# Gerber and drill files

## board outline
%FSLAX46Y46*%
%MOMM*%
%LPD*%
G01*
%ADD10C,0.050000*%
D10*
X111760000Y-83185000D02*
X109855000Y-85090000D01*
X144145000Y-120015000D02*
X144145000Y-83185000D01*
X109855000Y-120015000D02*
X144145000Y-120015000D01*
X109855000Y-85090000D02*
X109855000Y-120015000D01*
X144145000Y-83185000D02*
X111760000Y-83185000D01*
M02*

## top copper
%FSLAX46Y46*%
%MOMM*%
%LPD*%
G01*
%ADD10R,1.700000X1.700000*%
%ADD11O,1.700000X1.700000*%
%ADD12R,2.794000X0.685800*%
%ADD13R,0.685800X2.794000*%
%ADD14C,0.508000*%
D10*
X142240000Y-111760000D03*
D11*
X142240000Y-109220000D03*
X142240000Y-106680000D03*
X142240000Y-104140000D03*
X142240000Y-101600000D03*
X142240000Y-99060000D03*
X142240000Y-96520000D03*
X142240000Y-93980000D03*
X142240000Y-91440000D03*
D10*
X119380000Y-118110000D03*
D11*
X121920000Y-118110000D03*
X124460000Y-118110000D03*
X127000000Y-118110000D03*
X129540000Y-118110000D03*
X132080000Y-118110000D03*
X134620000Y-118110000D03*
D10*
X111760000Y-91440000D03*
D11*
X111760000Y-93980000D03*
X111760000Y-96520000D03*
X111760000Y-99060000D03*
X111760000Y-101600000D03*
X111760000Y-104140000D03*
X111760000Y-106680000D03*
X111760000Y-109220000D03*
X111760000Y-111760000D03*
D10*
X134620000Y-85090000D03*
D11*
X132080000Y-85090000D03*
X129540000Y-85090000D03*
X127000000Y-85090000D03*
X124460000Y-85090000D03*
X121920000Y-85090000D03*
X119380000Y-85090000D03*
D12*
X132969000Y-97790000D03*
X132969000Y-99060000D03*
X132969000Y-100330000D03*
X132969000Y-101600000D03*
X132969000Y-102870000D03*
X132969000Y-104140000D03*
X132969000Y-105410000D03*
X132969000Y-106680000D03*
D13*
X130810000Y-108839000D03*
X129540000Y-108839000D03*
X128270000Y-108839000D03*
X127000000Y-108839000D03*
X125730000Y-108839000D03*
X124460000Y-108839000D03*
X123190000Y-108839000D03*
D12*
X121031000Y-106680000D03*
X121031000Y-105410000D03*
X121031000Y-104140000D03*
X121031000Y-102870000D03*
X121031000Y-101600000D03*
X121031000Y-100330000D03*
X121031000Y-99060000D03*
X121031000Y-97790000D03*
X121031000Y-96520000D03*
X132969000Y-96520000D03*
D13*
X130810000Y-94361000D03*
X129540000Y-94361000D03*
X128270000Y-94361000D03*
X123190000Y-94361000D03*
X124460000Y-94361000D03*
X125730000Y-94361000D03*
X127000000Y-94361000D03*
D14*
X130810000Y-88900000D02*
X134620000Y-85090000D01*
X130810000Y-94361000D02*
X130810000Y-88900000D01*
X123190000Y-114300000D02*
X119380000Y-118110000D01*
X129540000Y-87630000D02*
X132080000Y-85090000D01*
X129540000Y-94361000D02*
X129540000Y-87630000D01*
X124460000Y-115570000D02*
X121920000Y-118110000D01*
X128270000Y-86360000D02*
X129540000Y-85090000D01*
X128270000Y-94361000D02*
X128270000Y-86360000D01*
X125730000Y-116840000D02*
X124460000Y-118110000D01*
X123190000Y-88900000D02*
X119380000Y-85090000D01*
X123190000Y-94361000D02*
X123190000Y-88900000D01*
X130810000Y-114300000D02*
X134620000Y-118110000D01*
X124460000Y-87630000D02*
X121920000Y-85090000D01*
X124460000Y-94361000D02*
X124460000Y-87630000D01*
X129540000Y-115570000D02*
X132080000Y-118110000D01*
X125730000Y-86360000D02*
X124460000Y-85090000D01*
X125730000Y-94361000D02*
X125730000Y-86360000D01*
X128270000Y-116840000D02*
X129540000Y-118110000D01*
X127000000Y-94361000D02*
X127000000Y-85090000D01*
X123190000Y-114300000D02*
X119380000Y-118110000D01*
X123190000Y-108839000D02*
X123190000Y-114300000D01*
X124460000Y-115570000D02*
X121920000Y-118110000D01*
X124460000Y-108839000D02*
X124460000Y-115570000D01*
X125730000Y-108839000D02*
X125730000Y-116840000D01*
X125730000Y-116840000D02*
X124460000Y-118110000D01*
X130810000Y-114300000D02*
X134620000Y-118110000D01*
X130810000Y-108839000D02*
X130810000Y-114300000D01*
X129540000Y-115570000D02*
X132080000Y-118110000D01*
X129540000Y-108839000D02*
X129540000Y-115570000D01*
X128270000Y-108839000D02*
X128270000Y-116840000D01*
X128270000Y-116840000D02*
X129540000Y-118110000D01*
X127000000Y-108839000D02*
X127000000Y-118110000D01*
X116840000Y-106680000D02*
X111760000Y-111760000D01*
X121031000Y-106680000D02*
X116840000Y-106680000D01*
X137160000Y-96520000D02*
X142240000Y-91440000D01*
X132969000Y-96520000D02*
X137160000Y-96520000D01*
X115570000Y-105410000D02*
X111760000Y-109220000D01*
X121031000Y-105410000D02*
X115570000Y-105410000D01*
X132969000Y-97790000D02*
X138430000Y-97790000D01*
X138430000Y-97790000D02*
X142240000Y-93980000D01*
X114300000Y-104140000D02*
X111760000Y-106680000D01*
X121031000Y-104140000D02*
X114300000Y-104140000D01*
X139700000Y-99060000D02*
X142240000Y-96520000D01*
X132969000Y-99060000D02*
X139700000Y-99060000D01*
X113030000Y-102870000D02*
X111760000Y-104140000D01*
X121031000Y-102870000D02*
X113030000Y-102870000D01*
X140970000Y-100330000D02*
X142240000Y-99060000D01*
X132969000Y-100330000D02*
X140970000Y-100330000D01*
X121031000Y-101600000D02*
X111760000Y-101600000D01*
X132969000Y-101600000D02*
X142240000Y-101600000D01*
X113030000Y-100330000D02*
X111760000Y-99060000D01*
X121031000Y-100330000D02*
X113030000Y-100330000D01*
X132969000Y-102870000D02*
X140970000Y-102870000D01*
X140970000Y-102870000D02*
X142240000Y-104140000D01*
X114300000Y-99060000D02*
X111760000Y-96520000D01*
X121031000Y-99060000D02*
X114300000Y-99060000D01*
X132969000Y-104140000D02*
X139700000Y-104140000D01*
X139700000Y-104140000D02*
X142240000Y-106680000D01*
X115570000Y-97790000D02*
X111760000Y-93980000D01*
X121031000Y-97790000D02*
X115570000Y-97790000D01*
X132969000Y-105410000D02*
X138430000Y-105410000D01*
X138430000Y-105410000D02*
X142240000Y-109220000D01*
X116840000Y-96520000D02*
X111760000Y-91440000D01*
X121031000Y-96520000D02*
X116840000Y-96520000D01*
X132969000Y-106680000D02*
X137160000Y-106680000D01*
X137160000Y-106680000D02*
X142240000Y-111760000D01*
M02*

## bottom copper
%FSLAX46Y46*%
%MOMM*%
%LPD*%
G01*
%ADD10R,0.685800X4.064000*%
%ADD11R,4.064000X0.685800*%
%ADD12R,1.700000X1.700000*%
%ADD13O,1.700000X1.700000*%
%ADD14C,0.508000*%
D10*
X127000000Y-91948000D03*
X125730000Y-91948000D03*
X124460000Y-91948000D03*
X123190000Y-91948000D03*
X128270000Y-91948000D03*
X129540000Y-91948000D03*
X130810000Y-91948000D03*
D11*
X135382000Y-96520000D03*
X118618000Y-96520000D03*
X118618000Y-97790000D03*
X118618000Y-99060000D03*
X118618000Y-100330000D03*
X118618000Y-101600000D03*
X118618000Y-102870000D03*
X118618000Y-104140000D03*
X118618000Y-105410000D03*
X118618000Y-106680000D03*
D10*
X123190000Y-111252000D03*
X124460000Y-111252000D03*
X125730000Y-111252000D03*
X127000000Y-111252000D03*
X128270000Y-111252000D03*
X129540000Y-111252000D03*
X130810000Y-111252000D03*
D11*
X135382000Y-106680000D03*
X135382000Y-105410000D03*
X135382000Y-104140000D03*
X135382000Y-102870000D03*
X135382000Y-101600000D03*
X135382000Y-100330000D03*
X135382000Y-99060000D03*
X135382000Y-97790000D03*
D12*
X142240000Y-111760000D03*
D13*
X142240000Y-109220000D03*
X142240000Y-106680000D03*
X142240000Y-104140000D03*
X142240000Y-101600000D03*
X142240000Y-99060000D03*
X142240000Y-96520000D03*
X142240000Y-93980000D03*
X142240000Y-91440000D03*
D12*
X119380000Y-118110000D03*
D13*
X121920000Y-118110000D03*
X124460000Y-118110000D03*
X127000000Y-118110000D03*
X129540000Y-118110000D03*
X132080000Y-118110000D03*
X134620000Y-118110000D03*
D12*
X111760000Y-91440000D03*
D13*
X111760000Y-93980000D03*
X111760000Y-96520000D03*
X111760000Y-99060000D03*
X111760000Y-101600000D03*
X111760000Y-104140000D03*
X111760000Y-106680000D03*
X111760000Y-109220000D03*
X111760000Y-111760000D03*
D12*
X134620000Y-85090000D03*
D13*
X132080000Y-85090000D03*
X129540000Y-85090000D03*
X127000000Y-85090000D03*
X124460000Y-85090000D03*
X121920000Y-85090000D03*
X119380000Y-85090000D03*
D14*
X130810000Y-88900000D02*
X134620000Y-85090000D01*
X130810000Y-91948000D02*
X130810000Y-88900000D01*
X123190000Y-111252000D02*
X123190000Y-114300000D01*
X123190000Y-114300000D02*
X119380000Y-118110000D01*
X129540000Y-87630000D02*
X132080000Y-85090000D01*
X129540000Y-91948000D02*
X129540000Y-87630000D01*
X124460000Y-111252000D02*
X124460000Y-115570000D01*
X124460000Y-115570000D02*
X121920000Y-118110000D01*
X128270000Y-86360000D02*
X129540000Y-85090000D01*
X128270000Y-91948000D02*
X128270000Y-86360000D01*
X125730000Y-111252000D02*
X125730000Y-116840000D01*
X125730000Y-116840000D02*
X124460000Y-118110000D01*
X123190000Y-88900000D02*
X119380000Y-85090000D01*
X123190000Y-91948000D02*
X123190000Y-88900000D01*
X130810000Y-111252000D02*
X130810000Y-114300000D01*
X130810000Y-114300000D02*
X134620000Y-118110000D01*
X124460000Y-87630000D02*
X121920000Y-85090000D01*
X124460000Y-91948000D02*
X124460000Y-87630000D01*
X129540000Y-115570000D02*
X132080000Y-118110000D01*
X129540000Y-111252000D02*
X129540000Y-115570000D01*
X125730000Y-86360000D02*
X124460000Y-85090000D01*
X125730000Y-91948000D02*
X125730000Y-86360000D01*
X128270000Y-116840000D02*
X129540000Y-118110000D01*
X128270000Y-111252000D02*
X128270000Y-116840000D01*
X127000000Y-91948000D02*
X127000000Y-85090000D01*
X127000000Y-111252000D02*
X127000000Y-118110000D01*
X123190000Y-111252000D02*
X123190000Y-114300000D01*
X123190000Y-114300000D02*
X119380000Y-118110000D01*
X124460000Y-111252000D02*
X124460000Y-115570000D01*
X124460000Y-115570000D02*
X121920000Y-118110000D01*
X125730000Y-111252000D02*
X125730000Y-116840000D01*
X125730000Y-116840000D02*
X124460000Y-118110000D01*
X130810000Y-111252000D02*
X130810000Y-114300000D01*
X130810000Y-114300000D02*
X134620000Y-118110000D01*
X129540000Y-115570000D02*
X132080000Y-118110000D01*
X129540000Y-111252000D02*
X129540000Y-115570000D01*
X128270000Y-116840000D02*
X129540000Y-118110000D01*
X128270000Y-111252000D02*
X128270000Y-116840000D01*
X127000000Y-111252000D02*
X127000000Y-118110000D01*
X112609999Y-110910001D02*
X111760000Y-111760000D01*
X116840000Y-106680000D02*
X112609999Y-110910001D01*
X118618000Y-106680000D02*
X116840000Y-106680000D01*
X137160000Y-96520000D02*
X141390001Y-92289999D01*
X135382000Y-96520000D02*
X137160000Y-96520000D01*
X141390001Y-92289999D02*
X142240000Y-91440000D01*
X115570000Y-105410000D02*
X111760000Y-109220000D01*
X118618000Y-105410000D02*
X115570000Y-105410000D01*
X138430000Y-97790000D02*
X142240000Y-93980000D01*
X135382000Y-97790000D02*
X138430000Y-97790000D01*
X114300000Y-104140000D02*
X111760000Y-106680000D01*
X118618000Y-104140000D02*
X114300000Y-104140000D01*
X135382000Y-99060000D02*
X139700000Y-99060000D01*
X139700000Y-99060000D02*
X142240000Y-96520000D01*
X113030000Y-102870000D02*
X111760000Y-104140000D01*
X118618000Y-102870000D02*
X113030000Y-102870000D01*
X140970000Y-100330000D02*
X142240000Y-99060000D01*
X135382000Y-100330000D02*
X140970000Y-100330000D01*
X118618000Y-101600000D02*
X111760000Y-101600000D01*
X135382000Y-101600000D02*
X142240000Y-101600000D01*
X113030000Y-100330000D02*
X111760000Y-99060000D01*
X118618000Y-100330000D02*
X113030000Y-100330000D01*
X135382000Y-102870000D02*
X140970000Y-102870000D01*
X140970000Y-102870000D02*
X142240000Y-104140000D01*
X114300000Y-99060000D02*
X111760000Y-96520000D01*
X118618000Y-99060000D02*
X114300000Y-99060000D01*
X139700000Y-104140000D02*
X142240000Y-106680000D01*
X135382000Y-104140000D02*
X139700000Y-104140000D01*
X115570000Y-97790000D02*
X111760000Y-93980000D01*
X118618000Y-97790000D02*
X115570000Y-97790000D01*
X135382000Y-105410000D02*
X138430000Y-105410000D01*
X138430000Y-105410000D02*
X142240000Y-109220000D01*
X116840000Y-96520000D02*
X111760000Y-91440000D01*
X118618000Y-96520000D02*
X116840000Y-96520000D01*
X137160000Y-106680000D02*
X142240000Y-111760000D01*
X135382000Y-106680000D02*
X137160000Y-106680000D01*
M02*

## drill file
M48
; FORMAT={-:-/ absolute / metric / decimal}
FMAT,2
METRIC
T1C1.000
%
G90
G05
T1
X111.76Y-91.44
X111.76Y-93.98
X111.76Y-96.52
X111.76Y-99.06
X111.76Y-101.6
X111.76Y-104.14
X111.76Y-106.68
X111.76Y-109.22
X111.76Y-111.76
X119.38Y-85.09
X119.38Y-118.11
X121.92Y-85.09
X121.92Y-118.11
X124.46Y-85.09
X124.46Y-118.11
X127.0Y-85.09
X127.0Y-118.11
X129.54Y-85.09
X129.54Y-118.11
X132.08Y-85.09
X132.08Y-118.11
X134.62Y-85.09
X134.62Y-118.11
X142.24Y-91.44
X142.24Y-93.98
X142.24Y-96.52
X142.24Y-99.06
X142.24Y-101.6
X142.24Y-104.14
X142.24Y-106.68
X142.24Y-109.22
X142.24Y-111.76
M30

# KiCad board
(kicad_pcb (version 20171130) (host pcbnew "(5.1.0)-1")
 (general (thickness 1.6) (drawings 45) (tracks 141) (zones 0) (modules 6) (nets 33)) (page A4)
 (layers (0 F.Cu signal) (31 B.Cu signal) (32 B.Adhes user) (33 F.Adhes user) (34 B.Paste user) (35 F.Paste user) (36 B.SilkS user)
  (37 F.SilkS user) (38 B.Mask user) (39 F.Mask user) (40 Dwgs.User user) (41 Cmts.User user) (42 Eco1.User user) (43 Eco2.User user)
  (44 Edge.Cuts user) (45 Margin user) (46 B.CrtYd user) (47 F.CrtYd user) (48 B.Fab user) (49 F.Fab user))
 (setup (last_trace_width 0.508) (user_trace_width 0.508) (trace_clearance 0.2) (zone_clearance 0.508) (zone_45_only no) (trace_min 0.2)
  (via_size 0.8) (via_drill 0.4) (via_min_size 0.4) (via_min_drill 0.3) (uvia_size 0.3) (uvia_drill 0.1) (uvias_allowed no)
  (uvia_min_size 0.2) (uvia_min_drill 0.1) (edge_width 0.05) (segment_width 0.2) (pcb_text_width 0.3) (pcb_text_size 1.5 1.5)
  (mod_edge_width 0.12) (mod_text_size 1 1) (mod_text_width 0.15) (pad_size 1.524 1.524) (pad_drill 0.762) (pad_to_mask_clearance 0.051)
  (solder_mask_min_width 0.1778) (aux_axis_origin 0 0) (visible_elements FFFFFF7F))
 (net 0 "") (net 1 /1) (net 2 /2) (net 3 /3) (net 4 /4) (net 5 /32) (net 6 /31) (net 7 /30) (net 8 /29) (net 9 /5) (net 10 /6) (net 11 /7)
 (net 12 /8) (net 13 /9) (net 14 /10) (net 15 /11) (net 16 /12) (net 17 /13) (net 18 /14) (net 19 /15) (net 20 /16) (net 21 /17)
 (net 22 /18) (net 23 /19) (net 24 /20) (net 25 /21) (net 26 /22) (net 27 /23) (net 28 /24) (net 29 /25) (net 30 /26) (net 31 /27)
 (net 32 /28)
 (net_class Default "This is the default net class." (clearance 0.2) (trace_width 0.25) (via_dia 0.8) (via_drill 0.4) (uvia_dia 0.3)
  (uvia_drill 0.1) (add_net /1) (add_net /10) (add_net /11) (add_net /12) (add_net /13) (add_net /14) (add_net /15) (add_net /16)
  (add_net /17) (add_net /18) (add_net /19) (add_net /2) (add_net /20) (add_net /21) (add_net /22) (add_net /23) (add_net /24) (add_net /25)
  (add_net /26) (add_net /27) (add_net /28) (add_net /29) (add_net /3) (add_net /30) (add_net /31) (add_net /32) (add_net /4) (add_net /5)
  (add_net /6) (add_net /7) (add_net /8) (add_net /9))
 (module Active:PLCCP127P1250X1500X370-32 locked (layer B.Cu) (at 127 101.6 180)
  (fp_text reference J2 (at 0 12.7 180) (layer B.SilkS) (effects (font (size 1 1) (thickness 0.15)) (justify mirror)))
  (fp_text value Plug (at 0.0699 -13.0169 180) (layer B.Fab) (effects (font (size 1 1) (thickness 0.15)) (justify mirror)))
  (pad 1 smd rect (at 0 9.652 180) (size 0.6858 4.064) (layers B.Cu B.Paste B.Mask) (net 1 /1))
  (pad 2 smd rect (at 1.27 9.652 180) (size 0.6858 4.064) (layers B.Cu B.Paste B.Mask) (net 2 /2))
  (pad 3 smd rect (at 2.54 9.652 180) (size 0.6858 4.064) (layers B.Cu B.Paste B.Mask) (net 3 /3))
  (pad 4 smd rect (at 3.81 9.652 180) (size 0.6858 4.064) (layers B.Cu B.Paste B.Mask) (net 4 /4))
  (pad 32 smd rect (at -1.27 9.652 180) (size 0.6858 4.064) (layers B.Cu B.Paste B.Mask) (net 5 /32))
  (pad 31 smd rect (at -2.54 9.652 180) (size 0.6858 4.064) (layers B.Cu B.Paste B.Mask) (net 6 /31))
  (pad 30 smd rect (at -3.81 9.652 180) (size 0.6858 4.064) (layers B.Cu B.Paste B.Mask) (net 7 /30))
  (pad 29 smd rect (at -8.382 5.08 270) (size 0.6858 4.064) (layers B.Cu B.Paste B.Mask) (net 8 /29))
  (pad 5 smd rect (at 8.382 5.08 270) (size 0.6858 4.064) (layers B.Cu B.Paste B.Mask) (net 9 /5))
  (pad 6 smd rect (at 8.382 3.81 270) (size 0.6858 4.064) (layers B.Cu B.Paste B.Mask) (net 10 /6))
  (pad 7 smd rect (at 8.382 2.54 270) (size 0.6858 4.064) (layers B.Cu B.Paste B.Mask) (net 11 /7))
  (pad 8 smd rect (at 8.382 1.27 270) (size 0.6858 4.064) (layers B.Cu B.Paste B.Mask) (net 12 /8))
  (pad 9 smd rect (at 8.382 0 270) (size 0.6858 4.064) (layers B.Cu B.Paste B.Mask) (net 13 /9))
  (pad 10 smd rect (at 8.382 -1.27 270) (size 0.6858 4.064) (layers B.Cu B.Paste B.Mask) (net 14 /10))
  (pad 11 smd rect (at 8.382 -2.54 270) (size 0.6858 4.064) (layers B.Cu B.Paste B.Mask) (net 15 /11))
  (pad 12 smd rect (at 8.382 -3.81 270) (size 0.6858 4.064) (layers B.Cu B.Paste B.Mask) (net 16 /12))
  (pad 13 smd rect (at 8.382 -5.08 270) (size 0.6858 4.064) (layers B.Cu B.Paste B.Mask) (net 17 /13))
  (pad 14 smd rect (at 3.81 -9.652 180) (size 0.6858 4.064) (layers B.Cu B.Paste B.Mask) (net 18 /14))
  (pad 15 smd rect (at 2.54 -9.652 180) (size 0.6858 4.064) (layers B.Cu B.Paste B.Mask) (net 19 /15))
  (pad 16 smd rect (at 1.27 -9.652 180) (size 0.6858 4.064) (layers B.Cu B.Paste B.Mask) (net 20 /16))
  (pad 17 smd rect (at 0 -9.652 180) (size 0.6858 4.064) (layers B.Cu B.Paste B.Mask) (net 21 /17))
  (pad 18 smd rect (at -1.27 -9.652 180) (size 0.6858 4.064) (layers B.Cu B.Paste B.Mask) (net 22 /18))
  (pad 19 smd rect (at -2.54 -9.652 180) (size 0.6858 4.064) (layers B.Cu B.Paste B.Mask) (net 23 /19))
  (pad 20 smd rect (at -3.81 -9.652 180) (size 0.6858 4.064) (layers B.Cu B.Paste B.Mask) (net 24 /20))
  (pad 21 smd rect (at -8.382 -5.08 270) (size 0.6858 4.064) (layers B.Cu B.Paste B.Mask) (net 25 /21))
  (pad 22 smd rect (at -8.382 -3.81 270) (size 0.6858 4.064) (layers B.Cu B.Paste B.Mask) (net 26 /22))
  (pad 23 smd rect (at -8.382 -2.54 270) (size 0.6858 4.064) (layers B.Cu B.Paste B.Mask) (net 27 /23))
  (pad 24 smd rect (at -8.382 -1.27 270) (size 0.6858 4.064) (layers B.Cu B.Paste B.Mask) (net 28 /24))
  (pad 25 smd rect (at -8.382 0 270) (size 0.6858 4.064) (layers B.Cu B.Paste B.Mask) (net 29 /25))
  (pad 26 smd rect (at -8.382 1.27 270) (size 0.6858 4.064) (layers B.Cu B.Paste B.Mask) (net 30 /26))
  (pad 27 smd rect (at -8.382 2.54 270) (size 0.6858 4.064) (layers B.Cu B.Paste B.Mask) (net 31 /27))
  (pad 28 smd rect (at -8.382 3.81 270) (size 0.6858 4.064) (layers B.Cu B.Paste B.Mask) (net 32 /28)))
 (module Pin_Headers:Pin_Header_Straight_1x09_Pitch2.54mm (layer F.Cu) (at 142.24 111.76 180)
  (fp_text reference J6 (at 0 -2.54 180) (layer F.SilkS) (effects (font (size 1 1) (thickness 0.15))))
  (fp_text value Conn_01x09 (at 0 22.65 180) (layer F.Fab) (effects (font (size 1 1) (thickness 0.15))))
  (pad 1 thru_hole rect (at 0 0 180) (size 1.7 1.7) (drill 1) (layers *.Cu *.Mask) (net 25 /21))
  (pad 2 thru_hole oval (at 0 2.54 180) (size 1.7 1.7) (drill 1) (layers *.Cu *.Mask) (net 26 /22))
  (pad 3 thru_hole oval (at 0 5.08 180) (size 1.7 1.7) (drill 1) (layers *.Cu *.Mask) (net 27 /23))
  (pad 4 thru_hole oval (at 0 7.62 180) (size 1.7 1.7) (drill 1) (layers *.Cu *.Mask) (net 28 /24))
  (pad 5 thru_hole oval (at 0 10.16 180) (size 1.7 1.7) (drill 1) (layers *.Cu *.Mask) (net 29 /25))
  (pad 6 thru_hole oval (at 0 12.7 180) (size 1.7 1.7) (drill 1) (layers *.Cu *.Mask) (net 30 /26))
  (pad 7 thru_hole oval (at 0 15.24 180) (size 1.7 1.7) (drill 1) (layers *.Cu *.Mask) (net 31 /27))
  (pad 8 thru_hole oval (at 0 17.78 180) (size 1.7 1.7) (drill 1) (layers *.Cu *.Mask) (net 32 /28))
  (pad 9 thru_hole oval (at 0 20.32 180) (size 1.7 1.7) (drill 1) (layers *.Cu *.Mask) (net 8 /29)))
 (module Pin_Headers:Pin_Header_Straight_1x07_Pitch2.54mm (layer F.Cu) (at 119.38 118.11 90)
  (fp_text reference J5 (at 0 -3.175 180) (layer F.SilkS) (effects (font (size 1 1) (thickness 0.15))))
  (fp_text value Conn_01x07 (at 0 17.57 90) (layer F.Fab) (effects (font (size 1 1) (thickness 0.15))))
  (pad 1 thru_hole rect (at 0 0 90) (size 1.7 1.7) (drill 1) (layers *.Cu *.Mask) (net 18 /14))
  (pad 2 thru_hole oval (at 0 2.54 90) (size 1.7 1.7) (drill 1) (layers *.Cu *.Mask) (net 19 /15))
  (pad 3 thru_hole oval (at 0 5.08 90) (size 1.7 1.7) (drill 1) (layers *.Cu *.Mask) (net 20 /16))
  (pad 4 thru_hole oval (at 0 7.62 90) (size 1.7 1.7) (drill 1) (layers *.Cu *.Mask) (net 21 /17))
  (pad 5 thru_hole oval (at 0 10.16 90) (size 1.7 1.7) (drill 1) (layers *.Cu *.Mask) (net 22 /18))
  (pad 6 thru_hole oval (at 0 12.7 90) (size 1.7 1.7) (drill 1) (layers *.Cu *.Mask) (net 23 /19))
  (pad 7 thru_hole oval (at 0 15.24 90) (size 1.7 1.7) (drill 1) (layers *.Cu *.Mask) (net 24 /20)))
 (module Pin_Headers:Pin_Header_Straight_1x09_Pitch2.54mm (layer F.Cu) (at 111.76 91.44)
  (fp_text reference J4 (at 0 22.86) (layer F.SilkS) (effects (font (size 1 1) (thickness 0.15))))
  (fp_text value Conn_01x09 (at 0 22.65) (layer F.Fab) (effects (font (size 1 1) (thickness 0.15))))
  (pad 1 thru_hole rect (at 0 0) (size 1.7 1.7) (drill 1) (layers *.Cu *.Mask) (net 9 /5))
  (pad 2 thru_hole oval (at 0 2.54) (size 1.7 1.7) (drill 1) (layers *.Cu *.Mask) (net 10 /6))
  (pad 3 thru_hole oval (at 0 5.08) (size 1.7 1.7) (drill 1) (layers *.Cu *.Mask) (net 11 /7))
  (pad 4 thru_hole oval (at 0 7.62) (size 1.7 1.7) (drill 1) (layers *.Cu *.Mask) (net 12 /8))
  (pad 5 thru_hole oval (at 0 10.16) (size 1.7 1.7) (drill 1) (layers *.Cu *.Mask) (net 13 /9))
  (pad 6 thru_hole oval (at 0 12.7) (size 1.7 1.7) (drill 1) (layers *.Cu *.Mask) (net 14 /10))
  (pad 7 thru_hole oval (at 0 15.24) (size 1.7 1.7) (drill 1) (layers *.Cu *.Mask) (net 15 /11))
  (pad 8 thru_hole oval (at 0 17.78) (size 1.7 1.7) (drill 1) (layers *.Cu *.Mask) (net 16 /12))
  (pad 9 thru_hole oval (at 0 20.32) (size 1.7 1.7) (drill 1) (layers *.Cu *.Mask) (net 17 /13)))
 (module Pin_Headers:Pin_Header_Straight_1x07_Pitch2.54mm (layer F.Cu) (at 134.62 85.09 270)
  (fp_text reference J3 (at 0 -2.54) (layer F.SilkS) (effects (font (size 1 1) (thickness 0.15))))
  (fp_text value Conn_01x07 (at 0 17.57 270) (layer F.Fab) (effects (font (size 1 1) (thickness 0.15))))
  (pad 1 thru_hole rect (at 0 0 270) (size 1.7 1.7) (drill 1) (layers *.Cu *.Mask) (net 7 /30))
  (pad 2 thru_hole oval (at 0 2.54 270) (size 1.7 1.7) (drill 1) (layers *.Cu *.Mask) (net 6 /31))
  (pad 3 thru_hole oval (at 0 5.08 270) (size 1.7 1.7) (drill 1) (layers *.Cu *.Mask) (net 5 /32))
  (pad 4 thru_hole oval (at 0 7.62 270) (size 1.7 1.7) (drill 1) (layers *.Cu *.Mask) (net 1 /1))
  (pad 5 thru_hole oval (at 0 10.16 270) (size 1.7 1.7) (drill 1) (layers *.Cu *.Mask) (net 2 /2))
  (pad 6 thru_hole oval (at 0 12.7 270) (size 1.7 1.7) (drill 1) (layers *.Cu *.Mask) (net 3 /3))
  (pad 7 thru_hole oval (at 0 15.24 270) (size 1.7 1.7) (drill 1) (layers *.Cu *.Mask) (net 4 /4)))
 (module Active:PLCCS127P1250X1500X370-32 (layer F.Cu) (at 127 101.6)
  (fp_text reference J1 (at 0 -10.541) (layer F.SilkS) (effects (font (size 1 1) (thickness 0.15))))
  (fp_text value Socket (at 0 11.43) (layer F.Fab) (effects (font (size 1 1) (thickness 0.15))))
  (pad 28 smd rect (at 5.969 -3.81 90) (size 0.6858 2.794) (layers F.Cu F.Paste F.Mask) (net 32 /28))
  (pad 27 smd rect (at 5.969 -2.54 90) (size 0.6858 2.794) (layers F.Cu F.Paste F.Mask) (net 31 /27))
  (pad 26 smd rect (at 5.969 -1.27 90) (size 0.6858 2.794) (layers F.Cu F.Paste F.Mask) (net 30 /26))
  (pad 25 smd rect (at 5.969 0 90) (size 0.6858 2.794) (layers F.Cu F.Paste F.Mask) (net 29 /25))
  (pad 24 smd rect (at 5.969 1.27 90) (size 0.6858 2.794) (layers F.Cu F.Paste F.Mask) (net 28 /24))
  (pad 23 smd rect (at 5.969 2.54 90) (size 0.6858 2.794) (layers F.Cu F.Paste F.Mask) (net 27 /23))
  (pad 22 smd rect (at 5.969 3.81 90) (size 0.6858 2.794) (layers F.Cu F.Paste F.Mask) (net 26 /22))
  (pad 21 smd rect (at 5.969 5.08 90) (size 0.6858 2.794) (layers F.Cu F.Paste F.Mask) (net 25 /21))
  (pad 20 smd rect (at 3.81 7.239) (size 0.6858 2.794) (layers F.Cu F.Paste F.Mask) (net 24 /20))
  (pad 19 smd rect (at 2.54 7.239) (size 0.6858 2.794) (layers F.Cu F.Paste F.Mask) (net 23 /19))
  (pad 18 smd rect (at 1.27 7.239) (size 0.6858 2.794) (layers F.Cu F.Paste F.Mask) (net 22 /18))
  (pad 17 smd rect (at 0 7.239) (size 0.6858 2.794) (layers F.Cu F.Paste F.Mask) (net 21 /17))
  (pad 16 smd rect (at -1.27 7.239) (size 0.6858 2.794) (layers F.Cu F.Paste F.Mask) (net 20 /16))
  (pad 15 smd rect (at -2.54 7.239) (size 0.6858 2.794) (layers F.Cu F.Paste F.Mask) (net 19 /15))
  (pad 14 smd rect (at -3.81 7.239) (size 0.6858 2.794) (layers F.Cu F.Paste F.Mask) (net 18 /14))
  (pad 13 smd rect (at -5.969 5.08 90) (size 0.6858 2.794) (layers F.Cu F.Paste F.Mask) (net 17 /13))
  (pad 12 smd rect (at -5.969 3.81 90) (size 0.6858 2.794) (layers F.Cu F.Paste F.Mask) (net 16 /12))
  (pad 11 smd rect (at -5.969 2.54 90) (size 0.6858 2.794) (layers F.Cu F.Paste F.Mask) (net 15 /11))
  (pad 10 smd rect (at -5.969 1.27 90) (size 0.6858 2.794) (layers F.Cu F.Paste F.Mask) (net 14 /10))
  (pad 9 smd rect (at -5.969 0 90) (size 0.6858 2.794) (layers F.Cu F.Paste F.Mask) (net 13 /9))
  (pad 8 smd rect (at -5.969 -1.27 90) (size 0.6858 2.794) (layers F.Cu F.Paste F.Mask) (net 12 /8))
  (pad 7 smd rect (at -5.969 -2.54 90) (size 0.6858 2.794) (layers F.Cu F.Paste F.Mask) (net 11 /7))
  (pad 6 smd rect (at -5.969 -3.81 90) (size 0.6858 2.794) (layers F.Cu F.Paste F.Mask) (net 10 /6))
  (pad 5 smd rect (at -5.969 -5.08 90) (size 0.6858 2.794) (layers F.Cu F.Paste F.Mask) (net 9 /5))
  (pad 29 smd rect (at 5.969 -5.08 90) (size 0.6858 2.794) (layers F.Cu F.Paste F.Mask) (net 8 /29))
  (pad 30 smd rect (at 3.81 -7.239) (size 0.6858 2.794) (layers F.Cu F.Paste F.Mask) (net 7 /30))
  (pad 31 smd rect (at 2.54 -7.239) (size 0.6858 2.794) (layers F.Cu F.Paste F.Mask) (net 6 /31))
  (pad 32 smd rect (at 1.27 -7.239) (size 0.6858 2.794) (layers F.Cu F.Paste F.Mask) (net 5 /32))
  (pad 4 smd rect (at -3.81 -7.239) (size 0.6858 2.794) (layers F.Cu F.Paste F.Mask) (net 4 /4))
  (pad 3 smd rect (at -2.54 -7.239) (size 0.6858 2.794) (layers F.Cu F.Paste F.Mask) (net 3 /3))
  (pad 2 smd rect (at -1.27 -7.239) (size 0.6858 2.794) (layers F.Cu F.Paste F.Mask) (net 2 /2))
  (pad 1 smd rect (at 0 -7.239) (size 0.6858 2.794) (layers F.Cu F.Paste F.Mask) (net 1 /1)))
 (gr_line (start 111.76 83.185) (end 109.855 85.09) (layer Edge.Cuts) (width 0.05))
 (gr_line (start 144.145 120.015) (end 144.145 83.185) (layer Edge.Cuts) (width 0.05))
 (gr_line (start 109.855 120.015) (end 144.145 120.015) (layer Edge.Cuts) (width 0.05))
 (gr_line (start 109.855 85.09) (end 109.855 120.015) (layer Edge.Cuts) (width 0.05))
 (gr_line (start 144.145 83.185) (end 111.76 83.185) (layer Edge.Cuts) (width 0.05))
 (segment (start 130.81 88.9) (end 134.62 85.09) (width 0.508) (layer F.Cu) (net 7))
 (segment (start 130.81 94.361) (end 130.81 88.9) (width 0.508) (layer F.Cu) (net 7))
 (segment (start 130.81 88.9) (end 134.62 85.09) (width 0.508) (layer B.Cu) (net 7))
 (segment (start 130.81 91.948) (end 130.81 88.9) (width 0.508) (layer B.Cu) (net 7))
 (segment (start 123.19 114.3) (end 119.38 118.11) (width 0.508) (layer F.Cu) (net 18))
 (segment (start 123.19 111.252) (end 123.19 114.3) (width 0.508) (layer B.Cu) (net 18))
 (segment (start 123.19 114.3) (end 119.38 118.11) (width 0.508) (layer B.Cu) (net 18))
 (segment (start 129.54 87.63) (end 132.08 85.09) (width 0.508) (layer F.Cu) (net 6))
 (segment (start 129.54 94.361) (end 129.54 87.63) (width 0.508) (layer F.Cu) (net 6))
 (segment (start 129.54 87.63) (end 132.08 85.09) (width 0.508) (layer B.Cu) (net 6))
 (segment (start 129.54 91.948) (end 129.54 87.63) (width 0.508) (layer B.Cu) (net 6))
 (segment (start 124.46 111.252) (end 124.46 115.57) (width 0.508) (layer B.Cu) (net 19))
 (segment (start 124.46 115.57) (end 121.92 118.11) (width 0.508) (layer B.Cu) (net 19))
 (segment (start 124.46 115.57) (end 121.92 118.11) (width 0.508) (layer F.Cu) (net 19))
 (segment (start 128.27 86.36) (end 129.54 85.09) (width 0.508) (layer F.Cu) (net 5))
 (segment (start 128.27 94.361) (end 128.27 86.36) (width 0.508) (layer F.Cu) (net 5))
 (segment (start 128.27 86.36) (end 129.54 85.09) (width 0.508) (layer B.Cu) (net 5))
 (segment (start 128.27 91.948) (end 128.27 86.36) (width 0.508) (layer B.Cu) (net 5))
 (segment (start 125.73 116.84) (end 124.46 118.11) (width 0.508) (layer F.Cu) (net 20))
 (segment (start 125.73 111.252) (end 125.73 116.84) (width 0.508) (layer B.Cu) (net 20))
 (segment (start 125.73 116.84) (end 124.46 118.11) (width 0.508) (layer B.Cu) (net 20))
 (segment (start 123.19 88.9) (end 119.38 85.09) (width 0.508) (layer F.Cu) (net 4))
 (segment (start 123.19 94.361) (end 123.19 88.9) (width 0.508) (layer F.Cu) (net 4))
 (segment (start 123.19 88.9) (end 119.38 85.09) (width 0.508) (layer B.Cu) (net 4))
 (segment (start 123.19 91.948) (end 123.19 88.9) (width 0.508) (layer B.Cu) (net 4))
 (segment (start 130.81 114.3) (end 134.62 118.11) (width 0.508) (layer F.Cu) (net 24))
 (segment (start 130.81 111.252) (end 130.81 114.3) (width 0.508) (layer B.Cu) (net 24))
 (segment (start 130.81 114.3) (end 134.62 118.11) (width 0.508) (layer B.Cu) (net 24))
 (segment (start 124.46 87.63) (end 121.92 85.09) (width 0.508) (layer F.Cu) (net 3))
 (segment (start 124.46 94.361) (end 124.46 87.63) (width 0.508) (layer F.Cu) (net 3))
 (segment (start 124.46 87.63) (end 121.92 85.09) (width 0.508) (layer B.Cu) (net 3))
 (segment (start 124.46 91.948) (end 124.46 87.63) (width 0.508) (layer B.Cu) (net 3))
 (segment (start 129.54 115.57) (end 132.08 118.11) (width 0.508) (layer F.Cu) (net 23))
 (segment (start 129.54 115.57) (end 132.08 118.11) (width 0.508) (layer B.Cu) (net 23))
 (segment (start 129.54 111.252) (end 129.54 115.57) (width 0.508) (layer B.Cu) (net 23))
 (segment (start 125.73 86.36) (end 124.46 85.09) (width 0.508) (layer F.Cu) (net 2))
 (segment (start 125.73 94.361) (end 125.73 86.36) (width 0.508) (layer F.Cu) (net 2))
 (segment (start 125.73 86.36) (end 124.46 85.09) (width 0.508) (layer B.Cu) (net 2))
 (segment (start 125.73 91.948) (end 125.73 86.36) (width 0.508) (layer B.Cu) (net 2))
 (segment (start 128.27 116.84) (end 129.54 118.11) (width 0.508) (layer B.Cu) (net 22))
 (segment (start 128.27 111.252) (end 128.27 116.84) (width 0.508) (layer B.Cu) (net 22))
 (segment (start 128.27 116.84) (end 129.54 118.11) (width 0.508) (layer F.Cu) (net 22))
 (segment (start 127 94.361) (end 127 85.09) (width 0.508) (layer F.Cu) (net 1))
 (segment (start 127 91.948) (end 127 85.09) (width 0.508) (layer B.Cu) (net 1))
 (segment (start 127 111.252) (end 127 118.11) (width 0.508) (layer B.Cu) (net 21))
 (segment (start 123.19 114.3) (end 119.38 118.11) (width 0.508) (layer F.Cu) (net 18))
 (segment (start 123.19 108.839) (end 123.19 114.3) (width 0.508) (layer F.Cu) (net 18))
 (segment (start 123.19 111.252) (end 123.19 114.3) (width 0.508) (layer B.Cu) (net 18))
 (segment (start 123.19 114.3) (end 119.38 118.11) (width 0.508) (layer B.Cu) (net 18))
 (segment (start 124.46 111.252) (end 124.46 115.57) (width 0.508) (layer B.Cu) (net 19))
 (segment (start 124.46 115.57) (end 121.92 118.11) (width 0.508) (layer B.Cu) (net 19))
 (segment (start 124.46 115.57) (end 121.92 118.11) (width 0.508) (layer F.Cu) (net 19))
 (segment (start 124.46 108.839) (end 124.46 115.57) (width 0.508) (layer F.Cu) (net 19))
 (segment (start 125.73 108.839) (end 125.73 116.84) (width 0.508) (layer F.Cu) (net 20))
 (segment (start 125.73 116.84) (end 124.46 118.11) (width 0.508) (layer F.Cu) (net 20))
 (segment (start 125.73 111.252) (end 125.73 116.84) (width 0.508) (layer B.Cu) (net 20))
 (segment (start 125.73 116.84) (end 124.46 118.11) (width 0.508) (layer B.Cu) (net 20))
 (segment (start 130.81 114.3) (end 134.62 118.11) (width 0.508) (layer F.Cu) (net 24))
 (segment (start 130.81 108.839) (end 130.81 114.3) (width 0.508) (layer F.Cu) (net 24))
 (segment (start 130.81 111.252) (end 130.81 114.3) (width 0.508) (layer B.Cu) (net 24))
 (segment (start 130.81 114.3) (end 134.62 118.11) (width 0.508) (layer B.Cu) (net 24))
 (segment (start 129.54 115.57) (end 132.08 118.11) (width 0.508) (layer F.Cu) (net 23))
 (segment (start 129.54 108.839) (end 129.54 115.57) (width 0.508) (layer F.Cu) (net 23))
 (segment (start 129.54 115.57) (end 132.08 118.11) (width 0.508) (layer B.Cu) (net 23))
 (segment (start 129.54 111.252) (end 129.54 115.57) (width 0.508) (layer B.Cu) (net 23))
 (segment (start 128.27 116.84) (end 129.54 118.11) (width 0.508) (layer B.Cu) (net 22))
 (segment (start 128.27 111.252) (end 128.27 116.84) (width 0.508) (layer B.Cu) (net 22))
 (segment (start 128.27 108.839) (end 128.27 116.84) (width 0.508) (layer F.Cu) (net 22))
 (segment (start 128.27 116.84) (end 129.54 118.11) (width 0.508) (layer F.Cu) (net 22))
 (segment (start 127 111.252) (end 127 118.11) (width 0.508) (layer B.Cu) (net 21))
 (segment (start 127 108.839) (end 127 118.11) (width 0.508) (layer F.Cu) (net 21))
 (segment (start 116.84 106.68) (end 111.76 111.76) (width 0.508) (layer F.Cu) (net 17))
 (segment (start 121.031 106.68) (end 116.84 106.68) (width 0.508) (layer F.Cu) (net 17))
 (segment (start 112.609999 110.910001) (end 111.76 111.76) (width 0.508) (layer B.Cu) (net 17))
 (segment (start 116.84 106.68) (end 112.609999 110.910001) (width 0.508) (layer B.Cu) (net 17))
 (segment (start 118.618 106.68) (end 116.84 106.68) (width 0.508) (layer B.Cu) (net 17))
 (segment (start 137.16 96.52) (end 141.390001 92.289999) (width 0.508) (layer B.Cu) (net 8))
 (segment (start 135.382 96.52) (end 137.16 96.52) (width 0.508) (layer B.Cu) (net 8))
 (segment (start 141.390001 92.289999) (end 142.24 91.44) (width 0.508) (layer B.Cu) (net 8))
 (segment (start 137.16 96.52) (end 142.24 91.44) (width 0.508) (layer F.Cu) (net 8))
 (segment (start 132.969 96.52) (end 137.16 96.52) (width 0.508) (layer F.Cu) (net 8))
 (segment (start 115.57 105.41) (end 111.76 109.22) (width 0.508) (layer F.Cu) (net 16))
 (segment (start 121.031 105.41) (end 115.57 105.41) (width 0.508) (layer F.Cu) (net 16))
 (segment (start 115.57 105.41) (end 111.76 109.22) (width 0.508) (layer B.Cu) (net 16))
 (segment (start 118.618 105.41) (end 115.57 105.41) (width 0.508) (layer B.Cu) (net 16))
 (segment (start 132.969 97.79) (end 138.43 97.79) (width 0.508) (layer F.Cu) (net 32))
 (segment (start 138.43 97.79) (end 142.24 93.98) (width 0.508) (layer F.Cu) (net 32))
 (segment (start 138.43 97.79) (end 142.24 93.98) (width 0.508) (layer B.Cu) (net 32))
 (segment (start 135.382 97.79) (end 138.43 97.79) (width 0.508) (layer B.Cu) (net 32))
 (segment (start 114.3 104.14) (end 111.76 106.68) (width 0.508) (layer F.Cu) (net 15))
 (segment (start 121.031 104.14) (end 114.3 104.14) (width 0.508) (layer F.Cu) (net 15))
 (segment (start 114.3 104.14) (end 111.76 106.68) (width 0.508) (layer B.Cu) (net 15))
 (segment (start 118.618 104.14) (end 114.3 104.14) (width 0.508) (layer B.Cu) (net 15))
 (segment (start 135.382 99.06) (end 139.7 99.06) (width 0.508) (layer B.Cu) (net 31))
 (segment (start 139.7 99.06) (end 142.24 96.52) (width 0.508) (layer B.Cu) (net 31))
 (segment (start 139.7 99.06) (end 142.24 96.52) (width 0.508) (layer F.Cu) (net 31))
 (segment (start 132.969 99.06) (end 139.7 99.06) (width 0.508) (layer F.Cu) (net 31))
 (segment (start 113.03 102.87) (end 111.76 104.14) (width 0.508) (layer F.Cu) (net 14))
 (segment (start 121.031 102.87) (end 113.03 102.87) (width 0.508) (layer F.Cu) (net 14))
 (segment (start 113.03 102.87) (end 111.76 104.14) (width 0.508) (layer B.Cu) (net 14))
 (segment (start 118.618 102.87) (end 113.03 102.87) (width 0.508) (layer B.Cu) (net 14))
 (segment (start 140.97 100.33) (end 142.24 99.06) (width 0.508) (layer B.Cu) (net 30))
 (segment (start 135.382 100.33) (end 140.97 100.33) (width 0.508) (layer B.Cu) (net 30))
 (segment (start 140.97 100.33) (end 142.24 99.06) (width 0.508) (layer F.Cu) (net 30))
 (segment (start 132.969 100.33) (end 140.97 100.33) (width 0.508) (layer F.Cu) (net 30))
 (segment (start 121.031 101.6) (end 111.76 101.6) (width 0.508) (layer F.Cu) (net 13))
 (segment (start 118.618 101.6) (end 111.76 101.6) (width 0.508) (layer B.Cu) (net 13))
 (segment (start 132.969 101.6) (end 142.24 101.6) (width 0.508) (layer F.Cu) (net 29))
 (segment (start 135.382 101.6) (end 142.24 101.6) (width 0.508) (layer B.Cu) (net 29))
 (segment (start 113.03 100.33) (end 111.76 99.06) (width 0.508) (layer F.Cu) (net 12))
 (segment (start 121.031 100.33) (end 113.03 100.33) (width 0.508) (layer F.Cu) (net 12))
 (segment (start 113.03 100.33) (end 111.76 99.06) (width 0.508) (layer B.Cu) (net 12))
 (segment (start 118.618 100.33) (end 113.03 100.33) (width 0.508) (layer B.Cu) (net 12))
 (segment (start 132.969 102.87) (end 140.97 102.87) (width 0.508) (layer F.Cu) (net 28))
 (segment (start 140.97 102.87) (end 142.24 104.14) (width 0.508) (layer F.Cu) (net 28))
 (segment (start 135.382 102.87) (end 140.97 102.87) (width 0.508) (layer B.Cu) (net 28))
 (segment (start 140.97 102.87) (end 142.24 104.14) (width 0.508) (layer B.Cu) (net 28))
 (segment (start 114.3 99.06) (end 111.76 96.52) (width 0.508) (layer F.Cu) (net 11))
 (segment (start 121.031 99.06) (end 114.3 99.06) (width 0.508) (layer F.Cu) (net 11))
 (segment (start 114.3 99.06) (end 111.76 96.52) (width 0.508) (layer B.Cu) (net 11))
 (segment (start 118.618 99.06) (end 114.3 99.06) (width 0.508) (layer B.Cu) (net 11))
 (segment (start 139.7 104.14) (end 142.24 106.68) (width 0.508) (layer B.Cu) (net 27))
 (segment (start 135.382 104.14) (end 139.7 104.14) (width 0.508) (layer B.Cu) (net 27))
 (segment (start 132.969 104.14) (end 139.7 104.14) (width 0.508) (layer F.Cu) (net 27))
 (segment (start 139.7 104.14) (end 142.24 106.68) (width 0.508) (layer F.Cu) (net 27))
 (segment (start 115.57 97.79) (end 111.76 93.98) (width 0.508) (layer F.Cu) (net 10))
 (segment (start 121.031 97.79) (end 115.57 97.79) (width 0.508) (layer F.Cu) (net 10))
 (segment (start 115.57 97.79) (end 111.76 93.98) (width 0.508) (layer B.Cu) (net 10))
 (segment (start 118.618 97.79) (end 115.57 97.79) (width 0.508) (layer B.Cu) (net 10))
 (segment (start 135.382 105.41) (end 138.43 105.41) (width 0.508) (layer B.Cu) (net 26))
 (segment (start 138.43 105.41) (end 142.24 109.22) (width 0.508) (layer B.Cu) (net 26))
 (segment (start 132.969 105.41) (end 138.43 105.41) (width 0.508) (layer F.Cu) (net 26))
 (segment (start 138.43 105.41) (end 142.24 109.22) (width 0.508) (layer F.Cu) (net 26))
 (segment (start 116.84 96.52) (end 111.76 91.44) (width 0.508) (layer B.Cu) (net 9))
 (segment (start 118.618 96.52) (end 116.84 96.52) (width 0.508) (layer B.Cu) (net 9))
 (segment (start 116.84 96.52) (end 111.76 91.44) (width 0.508) (layer F.Cu) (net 9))
 (segment (start 121.031 96.52) (end 116.84 96.52) (width 0.508) (layer F.Cu) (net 9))
 (segment (start 132.969 106.68) (end 137.16 106.68) (width 0.508) (layer F.Cu) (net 25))
 (segment (start 137.16 106.68) (end 142.24 111.76) (width 0.508) (layer B.Cu) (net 25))
 (segment (start 135.382 106.68) (end 137.16 106.68) (width 0.508) (layer B.Cu) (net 25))
 (segment (start 137.16 106.68) (end 142.24 111.76) (width 0.508) (layer F.Cu) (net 25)))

